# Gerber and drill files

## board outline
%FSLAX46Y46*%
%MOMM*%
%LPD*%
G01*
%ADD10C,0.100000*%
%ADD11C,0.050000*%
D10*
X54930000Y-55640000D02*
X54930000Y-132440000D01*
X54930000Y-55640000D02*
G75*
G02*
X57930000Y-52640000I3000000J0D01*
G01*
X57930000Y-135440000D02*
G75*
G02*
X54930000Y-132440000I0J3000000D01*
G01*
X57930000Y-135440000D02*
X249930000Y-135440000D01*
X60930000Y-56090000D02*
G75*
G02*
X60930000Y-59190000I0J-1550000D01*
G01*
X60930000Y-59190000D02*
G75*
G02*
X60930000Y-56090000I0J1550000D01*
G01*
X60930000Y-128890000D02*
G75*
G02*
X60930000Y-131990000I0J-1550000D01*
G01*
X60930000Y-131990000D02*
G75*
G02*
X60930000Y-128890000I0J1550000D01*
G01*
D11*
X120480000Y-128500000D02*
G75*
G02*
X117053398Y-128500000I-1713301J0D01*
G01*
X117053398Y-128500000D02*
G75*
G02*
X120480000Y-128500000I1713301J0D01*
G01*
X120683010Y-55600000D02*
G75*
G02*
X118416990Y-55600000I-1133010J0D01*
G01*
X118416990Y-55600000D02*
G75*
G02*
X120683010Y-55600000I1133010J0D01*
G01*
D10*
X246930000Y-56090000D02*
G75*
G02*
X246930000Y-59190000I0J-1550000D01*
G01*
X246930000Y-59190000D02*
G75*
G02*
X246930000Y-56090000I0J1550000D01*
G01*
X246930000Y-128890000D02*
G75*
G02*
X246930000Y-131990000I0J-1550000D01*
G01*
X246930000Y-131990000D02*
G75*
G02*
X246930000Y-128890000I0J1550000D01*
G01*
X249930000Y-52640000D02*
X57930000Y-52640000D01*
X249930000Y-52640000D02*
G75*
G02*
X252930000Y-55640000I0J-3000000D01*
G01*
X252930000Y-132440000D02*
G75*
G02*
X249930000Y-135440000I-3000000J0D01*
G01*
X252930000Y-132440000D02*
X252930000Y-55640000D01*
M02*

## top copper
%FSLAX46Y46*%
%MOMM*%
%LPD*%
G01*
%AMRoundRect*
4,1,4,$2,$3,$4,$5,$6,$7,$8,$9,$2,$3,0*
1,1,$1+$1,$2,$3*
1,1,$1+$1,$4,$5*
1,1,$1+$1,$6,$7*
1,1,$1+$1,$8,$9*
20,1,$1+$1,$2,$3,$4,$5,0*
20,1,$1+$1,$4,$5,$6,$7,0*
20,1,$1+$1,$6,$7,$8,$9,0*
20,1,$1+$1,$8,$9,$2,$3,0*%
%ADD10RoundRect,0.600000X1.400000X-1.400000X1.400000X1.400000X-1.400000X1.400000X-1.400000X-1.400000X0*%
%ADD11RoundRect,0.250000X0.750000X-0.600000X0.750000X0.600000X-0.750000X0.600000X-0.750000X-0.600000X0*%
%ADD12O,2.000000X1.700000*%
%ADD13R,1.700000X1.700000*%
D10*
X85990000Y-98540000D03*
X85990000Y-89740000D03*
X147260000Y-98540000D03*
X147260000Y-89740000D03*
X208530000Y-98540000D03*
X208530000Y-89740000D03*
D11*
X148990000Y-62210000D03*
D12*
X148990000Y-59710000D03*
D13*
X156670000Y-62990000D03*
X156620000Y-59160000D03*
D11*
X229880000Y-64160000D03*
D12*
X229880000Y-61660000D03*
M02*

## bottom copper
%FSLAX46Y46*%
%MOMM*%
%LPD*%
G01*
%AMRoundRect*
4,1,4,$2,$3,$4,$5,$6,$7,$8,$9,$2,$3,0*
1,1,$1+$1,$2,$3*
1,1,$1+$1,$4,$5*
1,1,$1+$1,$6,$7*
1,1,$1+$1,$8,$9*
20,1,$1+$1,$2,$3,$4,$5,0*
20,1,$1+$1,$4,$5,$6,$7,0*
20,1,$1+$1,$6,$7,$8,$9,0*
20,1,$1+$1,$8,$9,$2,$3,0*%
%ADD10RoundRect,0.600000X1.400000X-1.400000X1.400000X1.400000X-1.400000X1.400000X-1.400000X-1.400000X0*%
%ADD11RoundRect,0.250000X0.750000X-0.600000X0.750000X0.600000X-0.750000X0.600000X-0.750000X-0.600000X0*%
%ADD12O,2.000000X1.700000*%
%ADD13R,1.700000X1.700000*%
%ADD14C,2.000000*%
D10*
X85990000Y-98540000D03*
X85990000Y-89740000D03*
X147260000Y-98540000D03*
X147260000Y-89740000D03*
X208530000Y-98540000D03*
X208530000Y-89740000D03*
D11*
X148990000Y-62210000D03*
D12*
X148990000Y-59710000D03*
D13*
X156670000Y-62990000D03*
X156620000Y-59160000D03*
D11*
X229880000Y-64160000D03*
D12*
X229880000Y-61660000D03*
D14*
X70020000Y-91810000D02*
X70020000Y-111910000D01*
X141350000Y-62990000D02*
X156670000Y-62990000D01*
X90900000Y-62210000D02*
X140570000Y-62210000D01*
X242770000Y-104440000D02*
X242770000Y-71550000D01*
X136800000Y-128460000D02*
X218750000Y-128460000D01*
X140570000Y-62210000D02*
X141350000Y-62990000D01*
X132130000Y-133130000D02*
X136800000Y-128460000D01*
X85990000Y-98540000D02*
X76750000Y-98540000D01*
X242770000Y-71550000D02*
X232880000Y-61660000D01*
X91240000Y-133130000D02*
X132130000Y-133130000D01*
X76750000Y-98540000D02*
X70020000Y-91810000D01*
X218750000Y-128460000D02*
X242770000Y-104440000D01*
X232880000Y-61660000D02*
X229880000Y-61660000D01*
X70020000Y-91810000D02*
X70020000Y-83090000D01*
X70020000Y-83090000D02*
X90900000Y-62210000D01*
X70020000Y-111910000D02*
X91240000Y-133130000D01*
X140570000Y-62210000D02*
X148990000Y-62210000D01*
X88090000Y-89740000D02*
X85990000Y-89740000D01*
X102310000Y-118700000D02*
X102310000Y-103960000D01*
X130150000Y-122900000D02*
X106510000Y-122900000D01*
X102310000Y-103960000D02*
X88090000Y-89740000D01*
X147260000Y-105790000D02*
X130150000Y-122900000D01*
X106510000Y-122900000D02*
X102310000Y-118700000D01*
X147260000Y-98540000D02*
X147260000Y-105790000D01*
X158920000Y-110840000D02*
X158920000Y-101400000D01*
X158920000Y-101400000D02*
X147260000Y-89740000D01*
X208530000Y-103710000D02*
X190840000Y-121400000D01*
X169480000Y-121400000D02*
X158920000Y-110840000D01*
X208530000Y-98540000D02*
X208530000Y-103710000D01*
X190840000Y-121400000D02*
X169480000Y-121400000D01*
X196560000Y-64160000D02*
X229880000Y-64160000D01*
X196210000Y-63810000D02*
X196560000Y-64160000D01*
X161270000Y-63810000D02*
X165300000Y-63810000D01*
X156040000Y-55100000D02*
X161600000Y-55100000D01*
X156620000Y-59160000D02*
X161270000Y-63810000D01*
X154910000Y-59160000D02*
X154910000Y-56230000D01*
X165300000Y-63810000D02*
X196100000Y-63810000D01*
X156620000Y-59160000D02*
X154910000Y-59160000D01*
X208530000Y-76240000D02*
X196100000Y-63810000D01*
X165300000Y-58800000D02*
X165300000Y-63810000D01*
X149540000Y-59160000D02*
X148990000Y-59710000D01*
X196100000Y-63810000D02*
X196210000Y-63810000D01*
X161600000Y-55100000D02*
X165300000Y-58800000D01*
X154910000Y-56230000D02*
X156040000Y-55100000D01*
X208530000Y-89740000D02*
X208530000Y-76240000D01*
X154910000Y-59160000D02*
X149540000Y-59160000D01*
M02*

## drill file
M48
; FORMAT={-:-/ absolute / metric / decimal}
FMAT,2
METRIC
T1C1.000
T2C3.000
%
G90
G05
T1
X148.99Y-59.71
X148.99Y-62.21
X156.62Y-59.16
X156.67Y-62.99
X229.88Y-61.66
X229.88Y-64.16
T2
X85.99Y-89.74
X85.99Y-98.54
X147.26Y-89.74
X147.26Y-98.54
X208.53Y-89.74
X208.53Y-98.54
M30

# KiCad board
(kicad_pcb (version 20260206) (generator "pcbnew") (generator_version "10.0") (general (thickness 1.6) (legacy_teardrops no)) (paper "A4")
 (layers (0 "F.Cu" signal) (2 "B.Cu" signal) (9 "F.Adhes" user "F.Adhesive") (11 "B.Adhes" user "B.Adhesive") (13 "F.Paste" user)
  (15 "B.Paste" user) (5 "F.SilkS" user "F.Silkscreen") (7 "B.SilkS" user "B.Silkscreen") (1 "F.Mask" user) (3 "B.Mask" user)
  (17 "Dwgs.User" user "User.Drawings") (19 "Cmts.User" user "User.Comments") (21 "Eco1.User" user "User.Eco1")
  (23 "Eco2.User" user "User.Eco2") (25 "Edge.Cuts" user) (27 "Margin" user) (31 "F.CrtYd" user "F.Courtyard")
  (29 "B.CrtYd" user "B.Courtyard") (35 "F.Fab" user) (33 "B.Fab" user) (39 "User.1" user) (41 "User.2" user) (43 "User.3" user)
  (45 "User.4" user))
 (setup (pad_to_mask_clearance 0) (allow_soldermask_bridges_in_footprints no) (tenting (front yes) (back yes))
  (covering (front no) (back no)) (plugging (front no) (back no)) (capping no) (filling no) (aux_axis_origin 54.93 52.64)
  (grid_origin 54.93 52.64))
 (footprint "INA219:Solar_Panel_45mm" (layer "F.Cu") (at 85.99 94.14 90)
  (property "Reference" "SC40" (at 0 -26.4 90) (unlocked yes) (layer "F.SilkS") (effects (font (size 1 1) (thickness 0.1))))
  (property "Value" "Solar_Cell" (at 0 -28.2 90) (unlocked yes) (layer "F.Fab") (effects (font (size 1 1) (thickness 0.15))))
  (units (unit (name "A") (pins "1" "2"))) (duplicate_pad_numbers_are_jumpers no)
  (pad "1" thru_hole roundrect (at -4.4 0 90) (size 4 4) (drill 3) (layers "*.Cu" "*.Mask") (remove_unused_layers no)
   (roundrect_rratio 0.15) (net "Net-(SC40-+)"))
  (pad "2" thru_hole roundrect (at 4.4 0 90) (size 4 4) (drill 3) (layers "*.Cu" "*.Mask") (remove_unused_layers no) (roundrect_rratio 0.15)
   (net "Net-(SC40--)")))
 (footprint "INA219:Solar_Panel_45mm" (layer "F.Cu") (at 147.26 94.14 90)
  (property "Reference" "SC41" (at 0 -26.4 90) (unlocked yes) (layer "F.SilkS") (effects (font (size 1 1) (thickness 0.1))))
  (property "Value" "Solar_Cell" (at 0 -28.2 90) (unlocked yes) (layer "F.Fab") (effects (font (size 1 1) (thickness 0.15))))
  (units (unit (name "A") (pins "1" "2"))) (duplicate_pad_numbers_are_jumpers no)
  (pad "1" thru_hole roundrect (at -4.4 0 90) (size 4 4) (drill 3) (layers "*.Cu" "*.Mask") (remove_unused_layers no)
   (roundrect_rratio 0.15) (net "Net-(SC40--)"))
  (pad "2" thru_hole roundrect (at 4.4 0 90) (size 4 4) (drill 3) (layers "*.Cu" "*.Mask") (remove_unused_layers no) (roundrect_rratio 0.15)
   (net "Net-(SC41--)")))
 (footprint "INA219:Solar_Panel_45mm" (layer "F.Cu") (at 208.53 94.14 90)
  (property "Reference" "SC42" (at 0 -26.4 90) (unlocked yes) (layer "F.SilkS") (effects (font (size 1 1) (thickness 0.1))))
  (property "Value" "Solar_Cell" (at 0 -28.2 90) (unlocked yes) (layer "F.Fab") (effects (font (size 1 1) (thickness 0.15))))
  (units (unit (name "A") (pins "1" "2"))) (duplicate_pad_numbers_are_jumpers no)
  (pad "1" thru_hole roundrect (at -4.4 0 90) (size 4 4) (drill 3) (layers "*.Cu" "*.Mask") (remove_unused_layers no)
   (roundrect_rratio 0.15) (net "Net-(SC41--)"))
  (pad "2" thru_hole roundrect (at 4.4 0 90) (size 4 4) (drill 3) (layers "*.Cu" "*.Mask") (remove_unused_layers no) (roundrect_rratio 0.15)
   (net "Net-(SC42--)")))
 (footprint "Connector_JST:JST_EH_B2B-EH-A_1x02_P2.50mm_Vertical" (layer "B.Cu") (at 148.99 62.21 90)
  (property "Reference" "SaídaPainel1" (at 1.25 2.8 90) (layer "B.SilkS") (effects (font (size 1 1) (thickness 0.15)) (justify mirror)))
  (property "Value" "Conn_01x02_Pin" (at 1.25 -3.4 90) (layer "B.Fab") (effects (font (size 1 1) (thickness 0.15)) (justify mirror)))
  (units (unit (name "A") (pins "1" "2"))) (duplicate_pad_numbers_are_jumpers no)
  (pad "1" thru_hole roundrect (at 0 0 90) (size 1.7 2) (drill 1) (layers "*.Cu" "*.Mask") (remove_unused_layers no)
   (roundrect_rratio 0.147059) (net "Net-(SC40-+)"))
  (pad "2" thru_hole oval (at 2.5 0 90) (size 1.7 2) (drill 1) (layers "*.Cu" "*.Mask") (remove_unused_layers no) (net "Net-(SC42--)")))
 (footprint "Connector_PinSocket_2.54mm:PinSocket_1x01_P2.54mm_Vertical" (layer "B.Cu") (at 156.67 62.99 90)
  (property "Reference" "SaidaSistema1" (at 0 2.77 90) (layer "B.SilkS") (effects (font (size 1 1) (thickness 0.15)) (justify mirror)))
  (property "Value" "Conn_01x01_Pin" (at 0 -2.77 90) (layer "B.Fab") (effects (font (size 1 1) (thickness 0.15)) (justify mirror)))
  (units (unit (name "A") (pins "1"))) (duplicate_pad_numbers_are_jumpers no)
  (pad "1" thru_hole rect (at 0 0 90) (size 1.7 1.7) (drill 1) (layers "*.Cu" "*.Mask") (remove_unused_layers no) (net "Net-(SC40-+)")))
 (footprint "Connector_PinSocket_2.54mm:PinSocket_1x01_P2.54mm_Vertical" (layer "B.Cu") (at 156.62 59.16 90)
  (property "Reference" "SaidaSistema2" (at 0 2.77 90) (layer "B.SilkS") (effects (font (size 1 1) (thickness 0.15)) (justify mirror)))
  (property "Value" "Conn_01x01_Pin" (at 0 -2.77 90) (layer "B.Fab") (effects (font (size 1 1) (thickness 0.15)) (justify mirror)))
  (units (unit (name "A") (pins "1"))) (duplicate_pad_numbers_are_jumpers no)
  (pad "1" thru_hole rect (at 0 0 90) (size 1.7 1.7) (drill 1) (layers "*.Cu" "*.Mask") (remove_unused_layers no) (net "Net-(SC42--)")))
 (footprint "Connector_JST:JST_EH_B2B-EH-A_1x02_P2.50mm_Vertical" (layer "B.Cu") (at 229.88 64.16 90)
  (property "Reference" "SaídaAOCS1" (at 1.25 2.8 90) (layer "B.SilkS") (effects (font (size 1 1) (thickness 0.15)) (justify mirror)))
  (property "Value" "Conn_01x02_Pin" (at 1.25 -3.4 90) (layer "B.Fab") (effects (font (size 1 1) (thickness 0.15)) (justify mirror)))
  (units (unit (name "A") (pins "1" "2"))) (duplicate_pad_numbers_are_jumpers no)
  (pad "1" thru_hole roundrect (at 0 0 90) (size 1.7 2) (drill 1) (layers "*.Cu" "*.Mask") (remove_unused_layers no)
   (roundrect_rratio 0.147059) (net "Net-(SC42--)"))
  (pad "2" thru_hole oval (at 2.5 0 90) (size 1.7 2) (drill 1) (layers "*.Cu" "*.Mask") (remove_unused_layers no) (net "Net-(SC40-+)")))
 (gr_line (start 54.93 55.64) (end 54.93 132.44) (stroke (width 0) (type default)) (layer "Edge.Cuts"))
 (gr_arc (start 54.93 55.64) (mid 55.80868 53.51868) (end 57.93 52.64) (stroke (width 0) (type default)) (layer "Edge.Cuts"))
 (gr_arc (start 57.93 135.44) (mid 55.80868 134.56132) (end 54.93 132.44) (stroke (width 0) (type default)) (layer "Edge.Cuts"))
 (gr_line (start 57.93 135.44) (end 249.93 135.44) (stroke (width 0) (type default)) (layer "Edge.Cuts"))
 (gr_arc (start 60.93 56.09) (mid 62.48 57.64) (end 60.93 59.19) (stroke (width 0) (type default)) (layer "Edge.Cuts"))
 (gr_arc (start 60.93 59.19) (mid 59.38 57.64) (end 60.93 56.09) (stroke (width 0) (type default)) (layer "Edge.Cuts"))
 (gr_arc (start 60.93 128.89) (mid 62.48 130.44) (end 60.93 131.99) (stroke (width 0) (type default)) (layer "Edge.Cuts"))
 (gr_arc (start 60.93 131.99) (mid 59.38 130.44) (end 60.93 128.89) (stroke (width 0) (type default)) (layer "Edge.Cuts"))
 (gr_circle (center 118.766699 128.5) (end 120.316699 127.77) (stroke (width 0.05) (type default)) (fill no) (layer "Edge.Cuts"))
 (gr_circle (center 119.55 55.6) (end 120.68301 55.6) (stroke (width 0.05) (type solid)) (fill no) (layer "Edge.Cuts"))
 (gr_arc (start 246.93 56.09) (mid 248.48 57.64) (end 246.93 59.19) (stroke (width 0) (type default)) (layer "Edge.Cuts"))
 (gr_arc (start 246.93 59.19) (mid 245.38 57.64) (end 246.93 56.09) (stroke (width 0) (type default)) (layer "Edge.Cuts"))
 (gr_arc (start 246.93 128.89) (mid 248.48 130.44) (end 246.93 131.99) (stroke (width 0) (type default)) (layer "Edge.Cuts"))
 (gr_arc (start 246.93 131.99) (mid 245.38 130.44) (end 246.93 128.89) (stroke (width 0) (type default)) (layer "Edge.Cuts"))
 (gr_line (start 249.93 52.64) (end 57.93 52.64) (stroke (width 0) (type default)) (layer "Edge.Cuts"))
 (gr_arc (start 249.93 52.64) (mid 252.05132 53.51868) (end 252.93 55.64) (stroke (width 0) (type default)) (layer "Edge.Cuts"))
 (gr_arc (start 252.93 132.44) (mid 252.05132 134.56132) (end 249.93 135.44) (stroke (width 0) (type default)) (layer "Edge.Cuts"))
 (gr_line (start 252.93 132.44) (end 252.93 55.64) (stroke (width 0) (type default)) (layer "Edge.Cuts"))
 (segment (start 70.02 91.81) (end 70.02 111.91) (width 2) (layer "B.Cu") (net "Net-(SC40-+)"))
 (segment (start 141.35 62.99) (end 156.67 62.99) (width 2) (layer "B.Cu") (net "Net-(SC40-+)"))
 (segment (start 90.9 62.21) (end 140.57 62.21) (width 2) (layer "B.Cu") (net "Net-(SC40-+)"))
 (segment (start 242.77 104.44) (end 242.77 71.55) (width 2) (layer "B.Cu") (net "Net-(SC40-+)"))
 (segment (start 136.8 128.46) (end 218.75 128.46) (width 2) (layer "B.Cu") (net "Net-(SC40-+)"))
 (segment (start 140.57 62.21) (end 141.35 62.99) (width 2) (layer "B.Cu") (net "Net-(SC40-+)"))
 (segment (start 132.13 133.13) (end 136.8 128.46) (width 2) (layer "B.Cu") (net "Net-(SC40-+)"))
 (segment (start 85.99 98.54) (end 76.75 98.54) (width 2) (layer "B.Cu") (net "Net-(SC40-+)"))
 (segment (start 242.77 71.55) (end 232.88 61.66) (width 2) (layer "B.Cu") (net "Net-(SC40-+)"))
 (segment (start 91.24 133.13) (end 132.13 133.13) (width 2) (layer "B.Cu") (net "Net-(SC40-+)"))
 (segment (start 76.75 98.54) (end 70.02 91.81) (width 2) (layer "B.Cu") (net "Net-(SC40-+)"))
 (segment (start 218.75 128.46) (end 242.77 104.44) (width 2) (layer "B.Cu") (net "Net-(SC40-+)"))
 (segment (start 232.88 61.66) (end 229.88 61.66) (width 2) (layer "B.Cu") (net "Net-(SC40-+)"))
 (segment (start 70.02 91.81) (end 70.02 83.09) (width 2) (layer "B.Cu") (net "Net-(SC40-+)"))
 (segment (start 70.02 83.09) (end 90.9 62.21) (width 2) (layer "B.Cu") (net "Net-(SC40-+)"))
 (segment (start 70.02 111.91) (end 91.24 133.13) (width 2) (layer "B.Cu") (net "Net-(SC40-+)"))
 (segment (start 140.57 62.21) (end 148.99 62.21) (width 2) (layer "B.Cu") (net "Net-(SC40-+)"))
 (segment (start 88.09 89.74) (end 85.99 89.74) (width 2) (layer "B.Cu") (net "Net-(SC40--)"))
 (segment (start 102.31 118.7) (end 102.31 103.96) (width 2) (layer "B.Cu") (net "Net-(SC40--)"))
 (segment (start 130.15 122.9) (end 106.51 122.9) (width 2) (layer "B.Cu") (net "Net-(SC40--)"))
 (segment (start 102.31 103.96) (end 88.09 89.74) (width 2) (layer "B.Cu") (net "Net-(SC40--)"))
 (segment (start 147.26 105.79) (end 130.15 122.9) (width 2) (layer "B.Cu") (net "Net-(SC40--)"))
 (segment (start 106.51 122.9) (end 102.31 118.7) (width 2) (layer "B.Cu") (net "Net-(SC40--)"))
 (segment (start 147.26 98.54) (end 147.26 105.79) (width 2) (layer "B.Cu") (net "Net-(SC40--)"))
 (segment (start 158.92 110.84) (end 158.92 101.4) (width 2) (layer "B.Cu") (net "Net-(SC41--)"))
 (segment (start 158.92 101.4) (end 147.26 89.74) (width 2) (layer "B.Cu") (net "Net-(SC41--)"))
 (segment (start 208.53 103.71) (end 190.84 121.4) (width 2) (layer "B.Cu") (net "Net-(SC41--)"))
 (segment (start 169.48 121.4) (end 158.92 110.84) (width 2) (layer "B.Cu") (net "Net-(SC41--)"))
 (segment (start 208.53 98.54) (end 208.53 103.71) (width 2) (layer "B.Cu") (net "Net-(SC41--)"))
 (segment (start 190.84 121.4) (end 169.48 121.4) (width 2) (layer "B.Cu") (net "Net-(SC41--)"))
 (segment (start 196.56 64.16) (end 229.88 64.16) (width 2) (layer "B.Cu") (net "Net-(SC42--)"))
 (segment (start 196.21 63.81) (end 196.56 64.16) (width 2) (layer "B.Cu") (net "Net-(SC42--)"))
 (segment (start 161.27 63.81) (end 165.3 63.81) (width 2) (layer "B.Cu") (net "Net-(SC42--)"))
 (segment (start 156.04 55.1) (end 161.6 55.1) (width 2) (layer "B.Cu") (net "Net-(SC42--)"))
 (segment (start 156.62 59.16) (end 161.27 63.81) (width 2) (layer "B.Cu") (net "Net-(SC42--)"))
 (segment (start 154.91 59.16) (end 154.91 56.23) (width 2) (layer "B.Cu") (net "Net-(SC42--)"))
 (segment (start 165.3 63.81) (end 196.1 63.81) (width 2) (layer "B.Cu") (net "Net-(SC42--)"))
 (segment (start 156.62 59.16) (end 154.91 59.16) (width 2) (layer "B.Cu") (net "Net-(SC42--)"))
 (segment (start 208.53 76.24) (end 196.1 63.81) (width 2) (layer "B.Cu") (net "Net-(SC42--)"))
 (segment (start 165.3 58.8) (end 165.3 63.81) (width 2) (layer "B.Cu") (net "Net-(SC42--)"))
 (segment (start 149.54 59.16) (end 148.99 59.71) (width 2) (layer "B.Cu") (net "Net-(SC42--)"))
 (segment (start 196.1 63.81) (end 196.21 63.81) (width 2) (layer "B.Cu") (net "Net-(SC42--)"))
 (segment (start 161.6 55.1) (end 165.3 58.8) (width 2) (layer "B.Cu") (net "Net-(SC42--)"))
 (segment (start 154.91 56.23) (end 156.04 55.1) (width 2) (layer "B.Cu") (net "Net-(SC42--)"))
 (segment (start 208.53 89.74) (end 208.53 76.24) (width 2) (layer "B.Cu") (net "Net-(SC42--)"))
 (segment (start 154.91 59.16) (end 149.54 59.16) (width 2) (layer "B.Cu") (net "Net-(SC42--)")))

